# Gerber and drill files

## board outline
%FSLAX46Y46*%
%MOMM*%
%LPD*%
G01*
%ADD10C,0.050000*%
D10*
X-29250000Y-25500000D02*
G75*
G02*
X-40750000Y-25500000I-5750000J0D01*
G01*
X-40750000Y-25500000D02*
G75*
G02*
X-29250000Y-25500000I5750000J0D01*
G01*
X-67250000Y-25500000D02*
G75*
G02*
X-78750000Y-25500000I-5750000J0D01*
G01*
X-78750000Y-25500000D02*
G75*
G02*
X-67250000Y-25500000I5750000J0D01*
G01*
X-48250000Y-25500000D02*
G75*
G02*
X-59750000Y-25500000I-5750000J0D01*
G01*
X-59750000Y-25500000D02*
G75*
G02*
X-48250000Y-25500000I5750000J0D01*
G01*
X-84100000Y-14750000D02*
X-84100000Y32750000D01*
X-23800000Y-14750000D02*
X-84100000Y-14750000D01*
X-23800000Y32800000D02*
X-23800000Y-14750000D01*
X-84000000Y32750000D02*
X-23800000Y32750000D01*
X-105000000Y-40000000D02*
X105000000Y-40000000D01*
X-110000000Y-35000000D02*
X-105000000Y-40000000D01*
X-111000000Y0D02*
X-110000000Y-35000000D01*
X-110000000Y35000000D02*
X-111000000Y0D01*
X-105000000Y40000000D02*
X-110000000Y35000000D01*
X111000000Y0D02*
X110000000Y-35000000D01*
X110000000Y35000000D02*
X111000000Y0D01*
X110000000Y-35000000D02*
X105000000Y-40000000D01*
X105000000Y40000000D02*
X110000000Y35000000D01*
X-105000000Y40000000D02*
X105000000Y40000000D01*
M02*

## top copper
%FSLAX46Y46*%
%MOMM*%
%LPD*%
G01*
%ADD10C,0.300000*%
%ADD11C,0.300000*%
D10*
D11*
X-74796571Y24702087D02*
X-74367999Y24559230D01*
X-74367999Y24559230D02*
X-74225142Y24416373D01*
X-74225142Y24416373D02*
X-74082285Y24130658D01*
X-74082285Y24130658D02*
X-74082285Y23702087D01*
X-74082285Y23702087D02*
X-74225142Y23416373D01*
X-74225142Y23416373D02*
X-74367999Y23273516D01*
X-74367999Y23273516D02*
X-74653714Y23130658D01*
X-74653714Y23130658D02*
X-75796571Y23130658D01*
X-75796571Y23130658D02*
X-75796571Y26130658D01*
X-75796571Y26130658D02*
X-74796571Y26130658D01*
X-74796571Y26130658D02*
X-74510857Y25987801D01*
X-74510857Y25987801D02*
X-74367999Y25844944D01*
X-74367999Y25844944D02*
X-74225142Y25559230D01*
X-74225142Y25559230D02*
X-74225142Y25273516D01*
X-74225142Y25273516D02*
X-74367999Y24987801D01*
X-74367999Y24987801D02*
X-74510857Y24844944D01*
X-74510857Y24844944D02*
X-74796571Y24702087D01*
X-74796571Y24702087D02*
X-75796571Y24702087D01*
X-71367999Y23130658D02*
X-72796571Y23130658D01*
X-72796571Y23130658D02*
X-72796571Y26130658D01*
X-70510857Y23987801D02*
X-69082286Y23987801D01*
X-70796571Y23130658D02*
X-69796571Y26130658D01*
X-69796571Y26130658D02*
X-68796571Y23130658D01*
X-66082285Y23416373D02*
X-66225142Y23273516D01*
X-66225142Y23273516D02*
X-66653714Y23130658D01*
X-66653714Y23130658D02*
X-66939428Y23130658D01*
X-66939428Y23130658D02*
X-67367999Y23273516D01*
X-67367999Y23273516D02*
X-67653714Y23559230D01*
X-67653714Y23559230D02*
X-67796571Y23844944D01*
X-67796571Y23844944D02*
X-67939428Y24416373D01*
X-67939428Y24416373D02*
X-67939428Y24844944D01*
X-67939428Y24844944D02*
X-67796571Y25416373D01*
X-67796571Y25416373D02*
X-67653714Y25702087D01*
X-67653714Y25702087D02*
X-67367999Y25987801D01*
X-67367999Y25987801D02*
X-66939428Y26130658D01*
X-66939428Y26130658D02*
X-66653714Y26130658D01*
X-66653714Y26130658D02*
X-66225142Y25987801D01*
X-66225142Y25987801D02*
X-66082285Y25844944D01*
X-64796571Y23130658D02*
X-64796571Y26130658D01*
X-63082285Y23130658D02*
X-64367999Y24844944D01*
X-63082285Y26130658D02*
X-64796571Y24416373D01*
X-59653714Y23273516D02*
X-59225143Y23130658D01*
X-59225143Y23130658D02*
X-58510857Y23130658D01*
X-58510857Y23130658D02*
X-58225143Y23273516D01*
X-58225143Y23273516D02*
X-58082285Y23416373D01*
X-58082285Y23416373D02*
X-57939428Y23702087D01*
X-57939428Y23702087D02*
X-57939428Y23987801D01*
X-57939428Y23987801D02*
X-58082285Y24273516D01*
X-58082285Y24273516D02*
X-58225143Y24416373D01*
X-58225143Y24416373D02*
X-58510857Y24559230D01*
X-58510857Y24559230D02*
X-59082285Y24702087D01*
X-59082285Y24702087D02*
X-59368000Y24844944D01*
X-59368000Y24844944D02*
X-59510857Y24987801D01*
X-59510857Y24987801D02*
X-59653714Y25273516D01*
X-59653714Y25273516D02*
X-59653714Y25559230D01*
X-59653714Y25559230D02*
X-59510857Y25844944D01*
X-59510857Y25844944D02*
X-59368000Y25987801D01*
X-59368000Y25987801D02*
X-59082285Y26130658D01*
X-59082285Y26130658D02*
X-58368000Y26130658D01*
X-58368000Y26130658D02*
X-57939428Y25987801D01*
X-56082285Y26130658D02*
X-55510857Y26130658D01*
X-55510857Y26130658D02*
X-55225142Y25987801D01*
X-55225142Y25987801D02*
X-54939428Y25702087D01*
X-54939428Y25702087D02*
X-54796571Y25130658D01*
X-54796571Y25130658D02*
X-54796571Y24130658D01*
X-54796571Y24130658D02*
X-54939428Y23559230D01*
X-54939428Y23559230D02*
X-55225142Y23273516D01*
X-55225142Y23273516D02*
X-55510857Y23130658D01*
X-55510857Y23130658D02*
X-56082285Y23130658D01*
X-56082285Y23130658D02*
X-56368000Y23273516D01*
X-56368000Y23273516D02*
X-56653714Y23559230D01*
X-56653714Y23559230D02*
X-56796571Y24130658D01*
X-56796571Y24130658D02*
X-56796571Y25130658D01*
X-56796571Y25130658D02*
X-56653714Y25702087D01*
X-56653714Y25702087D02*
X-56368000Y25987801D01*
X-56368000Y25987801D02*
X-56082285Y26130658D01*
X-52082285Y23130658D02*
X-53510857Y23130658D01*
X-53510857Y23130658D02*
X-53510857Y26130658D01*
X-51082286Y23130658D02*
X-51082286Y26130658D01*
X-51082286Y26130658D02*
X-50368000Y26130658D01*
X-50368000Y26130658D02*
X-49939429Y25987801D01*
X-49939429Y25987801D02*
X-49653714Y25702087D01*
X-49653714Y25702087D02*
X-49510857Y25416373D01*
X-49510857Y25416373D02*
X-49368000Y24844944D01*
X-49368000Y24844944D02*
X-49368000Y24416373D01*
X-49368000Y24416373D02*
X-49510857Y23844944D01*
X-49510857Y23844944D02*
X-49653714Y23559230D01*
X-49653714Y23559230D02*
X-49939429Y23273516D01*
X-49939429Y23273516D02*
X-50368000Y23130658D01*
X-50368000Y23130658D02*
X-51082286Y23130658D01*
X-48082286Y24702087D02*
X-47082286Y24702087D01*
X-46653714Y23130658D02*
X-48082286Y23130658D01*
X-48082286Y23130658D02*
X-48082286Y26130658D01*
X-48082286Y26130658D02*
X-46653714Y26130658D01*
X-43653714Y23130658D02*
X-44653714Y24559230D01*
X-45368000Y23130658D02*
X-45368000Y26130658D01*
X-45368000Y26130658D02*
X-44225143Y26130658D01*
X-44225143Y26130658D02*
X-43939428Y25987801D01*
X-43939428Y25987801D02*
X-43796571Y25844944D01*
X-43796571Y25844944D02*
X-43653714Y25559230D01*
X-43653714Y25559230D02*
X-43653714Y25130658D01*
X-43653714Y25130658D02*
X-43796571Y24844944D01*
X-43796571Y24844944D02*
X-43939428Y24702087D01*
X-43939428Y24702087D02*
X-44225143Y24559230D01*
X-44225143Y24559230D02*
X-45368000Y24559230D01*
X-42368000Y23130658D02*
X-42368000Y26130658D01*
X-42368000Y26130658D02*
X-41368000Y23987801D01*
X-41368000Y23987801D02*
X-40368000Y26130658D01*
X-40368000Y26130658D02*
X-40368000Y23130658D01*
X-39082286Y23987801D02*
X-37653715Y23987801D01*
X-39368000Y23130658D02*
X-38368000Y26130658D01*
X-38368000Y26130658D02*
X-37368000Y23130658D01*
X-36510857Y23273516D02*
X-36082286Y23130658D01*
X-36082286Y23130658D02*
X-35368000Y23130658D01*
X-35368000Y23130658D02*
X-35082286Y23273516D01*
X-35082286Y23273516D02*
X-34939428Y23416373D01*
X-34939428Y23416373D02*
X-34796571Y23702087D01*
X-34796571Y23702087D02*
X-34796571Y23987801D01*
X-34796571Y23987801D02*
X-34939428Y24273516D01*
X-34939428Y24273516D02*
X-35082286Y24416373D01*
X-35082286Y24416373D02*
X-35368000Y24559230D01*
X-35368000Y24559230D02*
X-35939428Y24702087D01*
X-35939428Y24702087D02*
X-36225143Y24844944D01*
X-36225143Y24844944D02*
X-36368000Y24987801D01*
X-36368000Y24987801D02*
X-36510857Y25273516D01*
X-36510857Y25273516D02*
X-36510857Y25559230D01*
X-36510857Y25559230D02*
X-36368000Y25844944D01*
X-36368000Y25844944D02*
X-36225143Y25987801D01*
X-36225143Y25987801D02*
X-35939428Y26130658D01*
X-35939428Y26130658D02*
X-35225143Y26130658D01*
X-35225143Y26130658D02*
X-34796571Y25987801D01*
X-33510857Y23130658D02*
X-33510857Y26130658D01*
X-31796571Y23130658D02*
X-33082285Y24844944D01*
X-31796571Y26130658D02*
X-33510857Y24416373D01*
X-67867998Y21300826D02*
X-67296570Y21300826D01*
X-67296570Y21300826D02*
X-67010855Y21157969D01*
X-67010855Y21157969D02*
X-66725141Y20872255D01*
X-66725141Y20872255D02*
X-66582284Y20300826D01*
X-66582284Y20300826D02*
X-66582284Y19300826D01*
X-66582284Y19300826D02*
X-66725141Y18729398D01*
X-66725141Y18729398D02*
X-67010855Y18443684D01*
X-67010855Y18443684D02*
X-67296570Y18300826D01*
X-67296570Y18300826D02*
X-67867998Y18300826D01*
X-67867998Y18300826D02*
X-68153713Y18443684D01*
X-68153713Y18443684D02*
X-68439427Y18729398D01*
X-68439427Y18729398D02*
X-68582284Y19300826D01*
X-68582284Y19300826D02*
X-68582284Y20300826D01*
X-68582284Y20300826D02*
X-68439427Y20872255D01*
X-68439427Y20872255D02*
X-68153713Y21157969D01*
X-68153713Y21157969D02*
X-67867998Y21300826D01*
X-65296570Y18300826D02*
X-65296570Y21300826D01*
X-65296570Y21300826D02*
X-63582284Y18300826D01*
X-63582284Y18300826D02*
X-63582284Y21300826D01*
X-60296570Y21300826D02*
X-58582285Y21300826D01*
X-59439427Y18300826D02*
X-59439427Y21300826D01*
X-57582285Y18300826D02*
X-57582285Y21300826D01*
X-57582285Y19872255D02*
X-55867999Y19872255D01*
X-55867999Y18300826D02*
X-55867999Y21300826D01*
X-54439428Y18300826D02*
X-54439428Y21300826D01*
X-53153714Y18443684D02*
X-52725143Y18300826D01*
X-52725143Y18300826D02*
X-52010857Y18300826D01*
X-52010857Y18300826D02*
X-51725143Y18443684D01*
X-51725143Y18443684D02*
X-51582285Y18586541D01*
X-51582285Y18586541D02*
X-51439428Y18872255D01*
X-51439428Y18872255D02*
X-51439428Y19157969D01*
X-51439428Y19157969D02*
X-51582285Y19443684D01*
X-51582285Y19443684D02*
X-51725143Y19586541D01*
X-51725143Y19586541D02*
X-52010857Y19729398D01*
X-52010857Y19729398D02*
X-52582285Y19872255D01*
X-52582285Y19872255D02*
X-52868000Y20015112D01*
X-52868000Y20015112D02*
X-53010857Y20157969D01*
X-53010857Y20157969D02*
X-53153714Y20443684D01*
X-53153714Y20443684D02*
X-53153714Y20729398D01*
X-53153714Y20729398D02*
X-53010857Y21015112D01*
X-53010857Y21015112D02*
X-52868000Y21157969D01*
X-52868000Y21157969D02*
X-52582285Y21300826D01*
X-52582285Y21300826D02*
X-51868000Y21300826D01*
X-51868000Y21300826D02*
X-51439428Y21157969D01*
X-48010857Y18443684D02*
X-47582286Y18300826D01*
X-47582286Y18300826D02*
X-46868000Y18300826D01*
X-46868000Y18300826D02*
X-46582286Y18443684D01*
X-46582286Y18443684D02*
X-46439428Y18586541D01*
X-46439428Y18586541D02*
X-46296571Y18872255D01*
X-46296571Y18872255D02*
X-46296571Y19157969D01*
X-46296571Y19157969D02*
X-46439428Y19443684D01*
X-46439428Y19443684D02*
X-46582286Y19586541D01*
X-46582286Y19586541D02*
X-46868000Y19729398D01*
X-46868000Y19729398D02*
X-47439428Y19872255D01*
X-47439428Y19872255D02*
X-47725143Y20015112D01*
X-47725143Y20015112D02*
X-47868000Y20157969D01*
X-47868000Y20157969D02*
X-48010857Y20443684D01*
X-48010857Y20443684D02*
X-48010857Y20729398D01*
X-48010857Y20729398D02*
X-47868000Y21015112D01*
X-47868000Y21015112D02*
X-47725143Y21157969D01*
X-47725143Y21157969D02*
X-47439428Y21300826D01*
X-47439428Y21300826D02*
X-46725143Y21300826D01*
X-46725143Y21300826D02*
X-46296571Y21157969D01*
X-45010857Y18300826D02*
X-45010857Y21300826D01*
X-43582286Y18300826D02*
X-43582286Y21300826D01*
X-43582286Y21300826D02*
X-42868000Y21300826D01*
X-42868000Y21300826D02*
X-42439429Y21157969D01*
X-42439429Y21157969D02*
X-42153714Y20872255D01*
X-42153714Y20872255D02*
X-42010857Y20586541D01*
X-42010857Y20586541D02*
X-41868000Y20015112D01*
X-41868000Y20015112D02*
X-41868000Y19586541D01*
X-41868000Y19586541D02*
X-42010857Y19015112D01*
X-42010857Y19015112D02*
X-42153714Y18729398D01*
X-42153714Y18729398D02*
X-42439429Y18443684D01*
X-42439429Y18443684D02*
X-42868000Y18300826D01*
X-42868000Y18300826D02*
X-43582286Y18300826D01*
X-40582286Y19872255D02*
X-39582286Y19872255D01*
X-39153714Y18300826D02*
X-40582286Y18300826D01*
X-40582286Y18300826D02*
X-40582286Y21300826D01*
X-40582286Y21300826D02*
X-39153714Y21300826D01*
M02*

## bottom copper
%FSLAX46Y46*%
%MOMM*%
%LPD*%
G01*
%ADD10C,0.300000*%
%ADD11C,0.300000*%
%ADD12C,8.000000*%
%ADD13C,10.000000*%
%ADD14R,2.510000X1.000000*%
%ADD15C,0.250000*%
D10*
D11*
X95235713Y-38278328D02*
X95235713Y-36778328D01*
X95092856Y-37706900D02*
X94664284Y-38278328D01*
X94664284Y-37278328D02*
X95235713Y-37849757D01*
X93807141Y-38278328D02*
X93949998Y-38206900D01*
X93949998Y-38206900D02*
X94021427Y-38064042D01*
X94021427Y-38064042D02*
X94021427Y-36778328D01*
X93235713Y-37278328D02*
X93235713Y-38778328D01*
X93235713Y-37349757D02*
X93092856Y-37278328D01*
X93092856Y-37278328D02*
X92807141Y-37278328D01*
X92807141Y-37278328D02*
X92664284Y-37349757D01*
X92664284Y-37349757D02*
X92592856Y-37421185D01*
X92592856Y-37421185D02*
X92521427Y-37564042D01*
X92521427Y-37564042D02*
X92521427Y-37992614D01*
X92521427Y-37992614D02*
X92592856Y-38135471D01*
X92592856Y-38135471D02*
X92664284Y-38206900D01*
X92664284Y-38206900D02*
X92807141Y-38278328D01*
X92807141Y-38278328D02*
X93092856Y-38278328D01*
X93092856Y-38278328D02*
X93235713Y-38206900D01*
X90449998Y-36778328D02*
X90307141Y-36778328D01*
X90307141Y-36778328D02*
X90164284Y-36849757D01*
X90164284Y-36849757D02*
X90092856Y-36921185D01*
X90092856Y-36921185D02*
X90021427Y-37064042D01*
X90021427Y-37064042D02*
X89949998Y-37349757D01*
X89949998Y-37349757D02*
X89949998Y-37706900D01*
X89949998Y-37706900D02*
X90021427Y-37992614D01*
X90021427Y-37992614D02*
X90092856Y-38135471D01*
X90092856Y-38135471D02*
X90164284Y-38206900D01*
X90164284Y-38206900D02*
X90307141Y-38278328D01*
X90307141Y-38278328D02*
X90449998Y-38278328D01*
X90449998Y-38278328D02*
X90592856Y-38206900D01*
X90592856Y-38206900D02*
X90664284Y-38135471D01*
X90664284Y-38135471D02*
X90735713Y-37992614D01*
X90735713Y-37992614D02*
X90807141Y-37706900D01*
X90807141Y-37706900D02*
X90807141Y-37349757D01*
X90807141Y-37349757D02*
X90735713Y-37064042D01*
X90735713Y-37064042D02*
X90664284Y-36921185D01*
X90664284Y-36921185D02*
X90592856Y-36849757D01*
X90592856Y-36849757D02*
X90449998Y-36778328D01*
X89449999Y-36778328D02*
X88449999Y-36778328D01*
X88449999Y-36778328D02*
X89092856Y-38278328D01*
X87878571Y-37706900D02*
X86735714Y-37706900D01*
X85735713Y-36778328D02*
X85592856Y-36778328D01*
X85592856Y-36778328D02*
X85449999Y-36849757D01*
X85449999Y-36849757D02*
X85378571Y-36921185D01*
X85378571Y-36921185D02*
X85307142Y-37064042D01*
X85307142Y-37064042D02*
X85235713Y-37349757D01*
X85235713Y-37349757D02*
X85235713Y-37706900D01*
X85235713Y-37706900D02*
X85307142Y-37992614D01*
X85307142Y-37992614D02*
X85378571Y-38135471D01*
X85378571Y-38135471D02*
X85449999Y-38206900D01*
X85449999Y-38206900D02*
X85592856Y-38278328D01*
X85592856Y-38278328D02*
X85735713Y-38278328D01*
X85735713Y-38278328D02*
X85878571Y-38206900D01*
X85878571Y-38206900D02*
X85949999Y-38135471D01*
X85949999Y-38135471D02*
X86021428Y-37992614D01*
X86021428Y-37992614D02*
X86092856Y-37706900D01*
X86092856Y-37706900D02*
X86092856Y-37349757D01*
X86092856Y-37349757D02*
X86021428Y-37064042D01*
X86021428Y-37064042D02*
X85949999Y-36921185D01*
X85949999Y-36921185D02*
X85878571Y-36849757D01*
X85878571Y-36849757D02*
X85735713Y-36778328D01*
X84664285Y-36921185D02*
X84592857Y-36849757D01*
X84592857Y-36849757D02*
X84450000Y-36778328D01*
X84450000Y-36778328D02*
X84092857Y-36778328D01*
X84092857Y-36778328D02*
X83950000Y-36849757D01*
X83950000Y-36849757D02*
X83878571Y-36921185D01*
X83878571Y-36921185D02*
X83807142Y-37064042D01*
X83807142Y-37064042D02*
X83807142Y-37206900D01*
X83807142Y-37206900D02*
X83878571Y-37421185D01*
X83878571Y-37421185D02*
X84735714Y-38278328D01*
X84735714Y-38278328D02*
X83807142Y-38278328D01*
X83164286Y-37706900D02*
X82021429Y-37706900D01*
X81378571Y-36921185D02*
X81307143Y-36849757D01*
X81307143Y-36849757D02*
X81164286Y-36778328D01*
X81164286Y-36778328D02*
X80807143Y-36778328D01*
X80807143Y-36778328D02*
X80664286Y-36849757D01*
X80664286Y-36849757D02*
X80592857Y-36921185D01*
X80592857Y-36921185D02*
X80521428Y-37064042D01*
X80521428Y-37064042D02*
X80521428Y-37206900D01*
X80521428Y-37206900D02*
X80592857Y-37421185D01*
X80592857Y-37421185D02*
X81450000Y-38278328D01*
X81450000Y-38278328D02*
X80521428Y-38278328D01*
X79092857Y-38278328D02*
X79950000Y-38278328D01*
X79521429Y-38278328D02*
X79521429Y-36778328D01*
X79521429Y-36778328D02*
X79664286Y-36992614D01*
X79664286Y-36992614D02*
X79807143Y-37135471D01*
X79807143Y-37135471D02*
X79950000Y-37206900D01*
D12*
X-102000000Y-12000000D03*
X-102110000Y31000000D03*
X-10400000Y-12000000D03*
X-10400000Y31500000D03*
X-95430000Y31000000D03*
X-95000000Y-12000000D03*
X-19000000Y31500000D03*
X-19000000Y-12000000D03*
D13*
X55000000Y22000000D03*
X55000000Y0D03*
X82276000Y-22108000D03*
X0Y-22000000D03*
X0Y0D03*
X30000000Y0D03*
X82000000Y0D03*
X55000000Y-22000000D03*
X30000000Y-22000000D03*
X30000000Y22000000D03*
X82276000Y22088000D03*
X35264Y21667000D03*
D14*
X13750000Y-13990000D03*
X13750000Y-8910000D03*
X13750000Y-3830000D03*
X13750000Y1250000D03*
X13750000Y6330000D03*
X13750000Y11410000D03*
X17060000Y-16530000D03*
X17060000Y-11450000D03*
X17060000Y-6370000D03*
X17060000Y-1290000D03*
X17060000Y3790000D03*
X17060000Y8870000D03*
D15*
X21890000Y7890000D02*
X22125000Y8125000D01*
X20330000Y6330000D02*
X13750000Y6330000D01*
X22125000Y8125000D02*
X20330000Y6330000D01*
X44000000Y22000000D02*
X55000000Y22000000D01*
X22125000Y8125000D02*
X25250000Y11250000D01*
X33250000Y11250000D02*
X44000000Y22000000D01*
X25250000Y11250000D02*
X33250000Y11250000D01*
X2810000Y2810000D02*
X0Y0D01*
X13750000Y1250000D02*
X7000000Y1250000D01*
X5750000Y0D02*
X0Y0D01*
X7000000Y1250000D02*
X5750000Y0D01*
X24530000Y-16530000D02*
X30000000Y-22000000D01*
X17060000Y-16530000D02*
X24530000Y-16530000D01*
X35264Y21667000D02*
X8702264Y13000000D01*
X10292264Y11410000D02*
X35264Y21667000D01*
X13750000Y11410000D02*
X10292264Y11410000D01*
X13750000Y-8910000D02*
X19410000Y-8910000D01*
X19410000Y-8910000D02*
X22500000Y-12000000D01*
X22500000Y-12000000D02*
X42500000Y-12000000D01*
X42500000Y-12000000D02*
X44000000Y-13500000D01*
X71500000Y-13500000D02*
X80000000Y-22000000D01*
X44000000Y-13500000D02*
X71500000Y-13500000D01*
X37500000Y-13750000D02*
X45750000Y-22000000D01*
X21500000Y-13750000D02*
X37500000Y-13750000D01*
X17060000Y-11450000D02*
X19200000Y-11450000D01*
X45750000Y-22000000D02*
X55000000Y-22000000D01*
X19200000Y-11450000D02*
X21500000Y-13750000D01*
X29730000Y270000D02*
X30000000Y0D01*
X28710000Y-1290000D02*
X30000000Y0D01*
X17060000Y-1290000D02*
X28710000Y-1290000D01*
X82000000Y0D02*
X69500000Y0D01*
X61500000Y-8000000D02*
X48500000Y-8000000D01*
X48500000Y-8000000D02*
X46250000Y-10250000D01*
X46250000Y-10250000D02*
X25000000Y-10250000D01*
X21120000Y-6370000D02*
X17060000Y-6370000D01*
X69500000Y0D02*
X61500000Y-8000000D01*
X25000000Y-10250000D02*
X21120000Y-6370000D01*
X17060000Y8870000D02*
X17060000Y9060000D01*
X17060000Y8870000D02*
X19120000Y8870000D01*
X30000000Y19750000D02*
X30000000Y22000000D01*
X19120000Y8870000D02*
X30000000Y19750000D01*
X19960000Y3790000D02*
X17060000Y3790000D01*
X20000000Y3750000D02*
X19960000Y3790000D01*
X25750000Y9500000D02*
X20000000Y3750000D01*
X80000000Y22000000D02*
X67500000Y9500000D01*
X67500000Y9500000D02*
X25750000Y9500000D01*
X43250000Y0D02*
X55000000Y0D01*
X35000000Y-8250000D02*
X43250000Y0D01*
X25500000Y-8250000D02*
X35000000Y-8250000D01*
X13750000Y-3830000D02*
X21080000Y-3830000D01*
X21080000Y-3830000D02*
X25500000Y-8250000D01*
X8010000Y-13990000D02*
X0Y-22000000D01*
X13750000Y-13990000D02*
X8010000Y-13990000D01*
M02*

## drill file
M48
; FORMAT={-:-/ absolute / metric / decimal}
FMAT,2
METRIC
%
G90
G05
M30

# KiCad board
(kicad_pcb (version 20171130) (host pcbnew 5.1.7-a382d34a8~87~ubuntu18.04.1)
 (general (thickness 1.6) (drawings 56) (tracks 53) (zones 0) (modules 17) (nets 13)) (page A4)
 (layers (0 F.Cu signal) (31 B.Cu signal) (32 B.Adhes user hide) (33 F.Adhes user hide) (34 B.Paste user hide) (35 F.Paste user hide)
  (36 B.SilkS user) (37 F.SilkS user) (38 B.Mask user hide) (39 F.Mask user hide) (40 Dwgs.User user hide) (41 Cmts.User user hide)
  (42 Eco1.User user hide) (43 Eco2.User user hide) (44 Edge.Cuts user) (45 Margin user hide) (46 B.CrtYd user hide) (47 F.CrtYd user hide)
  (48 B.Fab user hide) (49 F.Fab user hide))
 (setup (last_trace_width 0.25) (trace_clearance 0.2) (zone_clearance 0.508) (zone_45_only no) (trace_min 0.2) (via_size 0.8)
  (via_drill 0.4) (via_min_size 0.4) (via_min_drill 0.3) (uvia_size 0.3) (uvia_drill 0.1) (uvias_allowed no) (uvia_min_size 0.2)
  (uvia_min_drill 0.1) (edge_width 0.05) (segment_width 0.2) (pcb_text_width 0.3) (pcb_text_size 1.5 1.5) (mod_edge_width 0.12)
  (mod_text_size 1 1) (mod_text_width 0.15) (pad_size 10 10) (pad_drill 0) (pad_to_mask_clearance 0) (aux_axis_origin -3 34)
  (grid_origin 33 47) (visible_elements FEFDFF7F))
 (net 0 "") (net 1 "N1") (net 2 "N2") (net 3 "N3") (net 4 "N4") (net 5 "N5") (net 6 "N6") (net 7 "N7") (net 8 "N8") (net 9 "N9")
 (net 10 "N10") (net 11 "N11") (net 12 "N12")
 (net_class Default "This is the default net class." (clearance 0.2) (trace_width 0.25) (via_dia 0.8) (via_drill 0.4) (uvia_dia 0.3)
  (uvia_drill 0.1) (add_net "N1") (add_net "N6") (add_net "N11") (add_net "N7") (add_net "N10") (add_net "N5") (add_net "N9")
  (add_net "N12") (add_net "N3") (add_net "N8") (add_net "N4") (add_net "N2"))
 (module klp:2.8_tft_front (layer F.Cu) (at -54 -9 270)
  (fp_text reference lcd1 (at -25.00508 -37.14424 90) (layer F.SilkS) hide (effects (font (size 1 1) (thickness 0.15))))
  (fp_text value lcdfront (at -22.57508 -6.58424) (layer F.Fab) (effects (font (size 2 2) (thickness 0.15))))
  (pad "" smd circle (at 21 48 270) (size 8 8) (layers B.Cu F.Paste F.Mask))
  (pad "" smd circle (at -22 48.11 270) (size 8 8) (layers B.Cu F.Paste F.Mask))
  (pad "" smd circle (at 21 -43.6 270) (size 8 8) (layers B.Cu F.Paste F.Mask))
  (pad "" smd circle (at -22.5 -43.6 270) (size 8 8) (layers B.Cu F.Paste F.Mask))
  (pad "" smd circle (at -22 41.43 270) (size 8 8) (layers B.Cu F.Paste F.Mask))
  (pad "" smd circle (at 21 41 270) (size 8 8) (layers B.Cu F.Paste F.Mask))
  (pad "" smd circle (at -22.5 -35 270) (size 8 8) (layers B.Cu F.Paste F.Mask))
  (pad "" smd circle (at 21 -35 270) (size 8 8) (layers B.Cu F.Paste F.Mask)))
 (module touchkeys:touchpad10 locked (layer B.Cu) (at 55 -22)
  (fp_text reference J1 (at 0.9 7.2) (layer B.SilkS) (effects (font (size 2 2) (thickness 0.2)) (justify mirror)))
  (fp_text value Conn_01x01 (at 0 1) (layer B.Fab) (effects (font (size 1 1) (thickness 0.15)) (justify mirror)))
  (pad 1 smd circle (at 0 0) (size 10 10) (layers B.Cu B.Paste B.Mask) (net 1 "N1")))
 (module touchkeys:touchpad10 (layer B.Cu) (at 55 0)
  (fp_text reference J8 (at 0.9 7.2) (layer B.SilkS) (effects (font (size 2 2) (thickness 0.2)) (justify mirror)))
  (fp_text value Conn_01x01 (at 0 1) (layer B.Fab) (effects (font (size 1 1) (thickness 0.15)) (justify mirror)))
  (pad 1 smd circle (at 0 0) (size 10 10) (layers B.Cu B.Paste B.Mask) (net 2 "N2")))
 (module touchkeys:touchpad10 (layer B.Cu) (at 82.276 22.108)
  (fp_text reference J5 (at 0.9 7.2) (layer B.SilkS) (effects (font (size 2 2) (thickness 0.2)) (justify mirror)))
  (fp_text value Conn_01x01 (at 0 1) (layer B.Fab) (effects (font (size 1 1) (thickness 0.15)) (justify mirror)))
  (pad 1 smd circle (at 0 0) (size 10 10) (layers B.Cu B.Paste B.Mask) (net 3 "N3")))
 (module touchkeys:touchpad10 (layer B.Cu) (at 0 22)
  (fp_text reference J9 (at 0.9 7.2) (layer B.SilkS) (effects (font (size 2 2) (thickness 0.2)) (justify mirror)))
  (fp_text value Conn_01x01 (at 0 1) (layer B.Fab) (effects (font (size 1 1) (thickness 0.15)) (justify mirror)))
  (pad 1 smd circle (at 0 0) (size 10 10) (layers B.Cu B.Paste B.Mask) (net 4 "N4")))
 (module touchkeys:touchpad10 (layer B.Cu) (at 0 0)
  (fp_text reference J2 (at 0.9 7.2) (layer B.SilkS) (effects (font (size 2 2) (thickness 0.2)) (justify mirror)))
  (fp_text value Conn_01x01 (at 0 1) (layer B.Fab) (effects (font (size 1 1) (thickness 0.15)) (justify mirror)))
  (pad 1 smd circle (at 0 0) (size 10 10) (layers B.Cu B.Paste B.Mask) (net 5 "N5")))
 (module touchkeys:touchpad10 (layer B.Cu) (at 30 0)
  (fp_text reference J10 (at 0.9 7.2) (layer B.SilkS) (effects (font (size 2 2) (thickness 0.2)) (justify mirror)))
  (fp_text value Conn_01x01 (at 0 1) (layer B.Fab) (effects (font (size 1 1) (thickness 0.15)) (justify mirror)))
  (pad 1 smd circle (at 0 0) (size 10 10) (layers B.Cu B.Paste B.Mask) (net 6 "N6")))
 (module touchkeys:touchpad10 (layer B.Cu) (at 82 0)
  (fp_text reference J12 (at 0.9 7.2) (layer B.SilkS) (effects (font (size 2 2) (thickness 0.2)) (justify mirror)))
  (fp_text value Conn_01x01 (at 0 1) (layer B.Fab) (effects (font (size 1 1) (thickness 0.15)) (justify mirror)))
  (pad 1 smd circle (at 0 0) (size 10 10) (layers B.Cu B.Paste B.Mask) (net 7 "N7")))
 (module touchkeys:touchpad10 (layer B.Cu) (at 55 22)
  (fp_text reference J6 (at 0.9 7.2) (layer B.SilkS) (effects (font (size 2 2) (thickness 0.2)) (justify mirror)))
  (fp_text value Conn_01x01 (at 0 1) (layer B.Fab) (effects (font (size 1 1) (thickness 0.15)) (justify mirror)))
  (pad 1 smd circle (at 0 0) (size 10 10) (layers B.Cu B.Paste B.Mask) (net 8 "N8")))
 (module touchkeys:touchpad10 (layer B.Cu) (at 30 22)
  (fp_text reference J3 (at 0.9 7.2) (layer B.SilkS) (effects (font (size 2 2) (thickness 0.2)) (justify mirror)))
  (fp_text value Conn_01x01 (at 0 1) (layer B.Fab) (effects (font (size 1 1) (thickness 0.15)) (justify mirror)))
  (pad 1 smd circle (at 0 0) (size 10 10) (layers B.Cu B.Paste B.Mask) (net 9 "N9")))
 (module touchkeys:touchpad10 (layer B.Cu) (at 30 -22)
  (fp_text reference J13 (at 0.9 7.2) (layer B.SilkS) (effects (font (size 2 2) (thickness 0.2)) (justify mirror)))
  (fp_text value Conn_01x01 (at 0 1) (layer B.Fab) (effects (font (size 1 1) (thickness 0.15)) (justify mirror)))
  (pad 1 smd circle (at 0 0) (size 10 10) (layers B.Cu B.Paste B.Mask) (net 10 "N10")))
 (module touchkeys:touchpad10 (layer B.Cu) (at 82.276 -22.088)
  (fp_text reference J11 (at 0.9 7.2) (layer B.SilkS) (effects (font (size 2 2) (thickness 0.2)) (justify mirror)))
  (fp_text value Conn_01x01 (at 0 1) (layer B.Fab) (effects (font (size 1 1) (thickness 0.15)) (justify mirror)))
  (pad 1 smd circle (at 0 0) (size 10 10) (layers B.Cu B.Paste B.Mask) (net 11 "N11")))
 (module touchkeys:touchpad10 (layer B.Cu) (at 0.035264 -21.667)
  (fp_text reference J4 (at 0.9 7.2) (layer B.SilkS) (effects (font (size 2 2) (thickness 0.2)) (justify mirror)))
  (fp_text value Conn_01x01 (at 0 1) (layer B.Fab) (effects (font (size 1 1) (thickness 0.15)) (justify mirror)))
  (pad 1 smd circle (at 0 0) (size 10 10) (layers B.Cu B.Paste B.Mask) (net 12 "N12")))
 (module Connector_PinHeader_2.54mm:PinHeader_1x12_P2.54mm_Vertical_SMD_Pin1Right (layer B.Cu) (at 15.405 2.56 180)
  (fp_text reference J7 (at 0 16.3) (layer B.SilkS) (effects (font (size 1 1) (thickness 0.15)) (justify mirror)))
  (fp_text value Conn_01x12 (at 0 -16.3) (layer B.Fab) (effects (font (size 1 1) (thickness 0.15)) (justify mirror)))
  (pad 11 smd rect (at 1.655 -11.43 180) (size 2.51 1) (layers B.Cu B.Paste B.Mask) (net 4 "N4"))
  (pad 9 smd rect (at 1.655 -6.35 180) (size 2.51 1) (layers B.Cu B.Paste B.Mask) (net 3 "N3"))
  (pad 7 smd rect (at 1.655 -1.27 180) (size 2.51 1) (layers B.Cu B.Paste B.Mask) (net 2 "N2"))
  (pad 5 smd rect (at 1.655 3.81 180) (size 2.51 1) (layers B.Cu B.Paste B.Mask) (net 5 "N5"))
  (pad 3 smd rect (at 1.655 8.89 180) (size 2.51 1) (layers B.Cu B.Paste B.Mask) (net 1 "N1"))
  (pad 1 smd rect (at 1.655 13.97 180) (size 2.51 1) (layers B.Cu B.Paste B.Mask) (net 12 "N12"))
  (pad 12 smd rect (at -1.655 -13.97 180) (size 2.51 1) (layers B.Cu B.Paste B.Mask) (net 9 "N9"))
  (pad 10 smd rect (at -1.655 -8.89 180) (size 2.51 1) (layers B.Cu B.Paste B.Mask) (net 8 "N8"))
  (pad 8 smd rect (at -1.655 -3.81 180) (size 2.51 1) (layers B.Cu B.Paste B.Mask) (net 7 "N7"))
  (pad 6 smd rect (at -1.655 1.27 180) (size 2.51 1) (layers B.Cu B.Paste B.Mask) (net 6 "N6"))
  (pad 4 smd rect (at -1.655 6.35 180) (size 2.51 1) (layers B.Cu B.Paste B.Mask) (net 11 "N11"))
  (pad 2 smd rect (at -1.655 11.43 180) (size 2.51 1) (layers B.Cu B.Paste B.Mask) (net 10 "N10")))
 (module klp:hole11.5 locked (layer F.Cu) (at -35 25.5)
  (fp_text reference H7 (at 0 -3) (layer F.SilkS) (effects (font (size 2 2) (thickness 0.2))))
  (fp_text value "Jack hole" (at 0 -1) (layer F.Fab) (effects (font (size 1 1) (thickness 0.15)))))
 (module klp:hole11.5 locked (layer F.Cu) (at -54 25.5)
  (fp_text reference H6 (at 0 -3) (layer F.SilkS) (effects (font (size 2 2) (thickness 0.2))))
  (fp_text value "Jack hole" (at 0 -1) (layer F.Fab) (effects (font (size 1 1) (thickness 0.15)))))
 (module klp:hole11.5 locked (layer F.Cu) (at -73 25.5)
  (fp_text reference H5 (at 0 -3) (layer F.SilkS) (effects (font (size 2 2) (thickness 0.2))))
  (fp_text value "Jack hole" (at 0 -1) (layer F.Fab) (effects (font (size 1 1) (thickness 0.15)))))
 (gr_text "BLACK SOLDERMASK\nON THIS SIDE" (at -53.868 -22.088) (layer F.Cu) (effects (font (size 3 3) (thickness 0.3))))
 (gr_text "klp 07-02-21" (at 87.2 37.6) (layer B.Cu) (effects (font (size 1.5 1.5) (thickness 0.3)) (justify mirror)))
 (gr_circle (center -35 25.5) (end -29.25 25.5) (layer Edge.Cuts) (width 0.05))
 (gr_circle (center -73 25.5) (end -67.25 25.5) (layer Edge.Cuts) (width 0.05))
 (gr_circle (center -54 25.5) (end -48.25 25.5) (layer Edge.Cuts) (width 0.05))
 (gr_line (start -84.1 14.75) (end -84.1 -32.75) (layer Edge.Cuts) (width 0.05))
 (gr_line (start -23.8 14.75) (end -84.1 14.75) (layer Edge.Cuts) (width 0.05))
 (gr_line (start -23.8 -32.8) (end -23.8 14.75) (layer Edge.Cuts) (width 0.05))
 (gr_line (start -84 -32.75) (end -23.8 -32.75) (layer Edge.Cuts) (width 0.05))
 (gr_line (start -105 40) (end 105 40) (layer Edge.Cuts) (width 0.05))
 (gr_line (start -110 35) (end -105 40) (layer Edge.Cuts) (width 0.05))
 (gr_line (start -111 0) (end -110 35) (layer Edge.Cuts) (width 0.05))
 (gr_line (start -110 -35) (end -111 0) (layer Edge.Cuts) (width 0.05))
 (gr_line (start -105 -40) (end -110 -35) (layer Edge.Cuts) (width 0.05))
 (gr_line (start 111 0) (end 110 35) (layer Edge.Cuts) (width 0.05))
 (gr_line (start 110 -35) (end 111 0) (layer Edge.Cuts) (width 0.05))
 (gr_line (start 110 35) (end 105 40) (layer Edge.Cuts) (width 0.05))
 (gr_line (start 105 -40) (end 110 -35) (layer Edge.Cuts) (width 0.05))
 (gr_line (start -105 -40) (end 105 -40) (layer Edge.Cuts) (width 0.05))
 (segment (start 21.89 -7.89) (end 22.125 -8.125) (width 0.25) (layer B.Cu) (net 1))
 (segment (start 20.33 -6.33) (end 13.75 -6.33) (width 0.25) (layer B.Cu) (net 1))
 (segment (start 22.125 -8.125) (end 20.33 -6.33) (width 0.25) (layer B.Cu) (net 1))
 (segment (start 44 -22) (end 55 -22) (width 0.25) (layer B.Cu) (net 1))
 (segment (start 22.125 -8.125) (end 25.25 -11.25) (width 0.25) (layer B.Cu) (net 1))
 (segment (start 33.25 -11.25) (end 44 -22) (width 0.25) (layer B.Cu) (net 1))
 (segment (start 25.25 -11.25) (end 33.25 -11.25) (width 0.25) (layer B.Cu) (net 1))
 (segment (start 2.81 -2.81) (end 0 0) (width 0.25) (layer B.Cu) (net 5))
 (segment (start 13.75 -1.25) (end 7 -1.25) (width 0.25) (layer B.Cu) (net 5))
 (segment (start 5.75 0) (end 0 0) (width 0.25) (layer B.Cu) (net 5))
 (segment (start 7 -1.25) (end 5.75 0) (width 0.25) (layer B.Cu) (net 5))
 (segment (start 24.53 16.53) (end 30 22) (width 0.25) (layer B.Cu) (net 9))
 (segment (start 17.06 16.53) (end 24.53 16.53) (width 0.25) (layer B.Cu) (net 9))
 (segment (start 0.035264 -21.667) (end 8.702264 -13) (width 0.25) (layer B.Cu) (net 12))
 (segment (start 10.292264 -11.41) (end 0.035264 -21.667) (width 0.25) (layer B.Cu) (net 12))
 (segment (start 13.75 -11.41) (end 10.292264 -11.41) (width 0.25) (layer B.Cu) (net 12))
 (segment (start 13.75 8.91) (end 19.41 8.91) (width 0.25) (layer B.Cu) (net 3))
 (segment (start 19.41 8.91) (end 22.5 12) (width 0.25) (layer B.Cu) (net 3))
 (segment (start 22.5 12) (end 42.5 12) (width 0.25) (layer B.Cu) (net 3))
 (segment (start 42.5 12) (end 44 13.5) (width 0.25) (layer B.Cu) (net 3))
 (segment (start 71.5 13.5) (end 80 22) (width 0.25) (layer B.Cu) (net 3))
 (segment (start 44 13.5) (end 71.5 13.5) (width 0.25) (layer B.Cu) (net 3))
 (segment (start 37.5 13.75) (end 45.75 22) (width 0.25) (layer B.Cu) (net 8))
 (segment (start 21.5 13.75) (end 37.5 13.75) (width 0.25) (layer B.Cu) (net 8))
 (segment (start 17.06 11.45) (end 19.2 11.45) (width 0.25) (layer B.Cu) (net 8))
 (segment (start 45.75 22) (end 55 22) (width 0.25) (layer B.Cu) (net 8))
 (segment (start 19.2 11.45) (end 21.5 13.75) (width 0.25) (layer B.Cu) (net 8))
 (segment (start 29.73 -0.27) (end 30 0) (width 0.25) (layer B.Cu) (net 6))
 (segment (start 28.71 1.29) (end 30 0) (width 0.25) (layer B.Cu) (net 6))
 (segment (start 17.06 1.29) (end 28.71 1.29) (width 0.25) (layer B.Cu) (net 6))
 (segment (start 82 0) (end 69.5 0) (width 0.25) (layer B.Cu) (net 7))
 (segment (start 61.5 8) (end 48.5 8) (width 0.25) (layer B.Cu) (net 7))
 (segment (start 48.5 8) (end 46.25 10.25) (width 0.25) (layer B.Cu) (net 7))
 (segment (start 46.25 10.25) (end 25 10.25) (width 0.25) (layer B.Cu) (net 7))
 (segment (start 21.12 6.37) (end 17.06 6.37) (width 0.25) (layer B.Cu) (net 7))
 (segment (start 69.5 0) (end 61.5 8) (width 0.25) (layer B.Cu) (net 7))
 (segment (start 25 10.25) (end 21.12 6.37) (width 0.25) (layer B.Cu) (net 7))
 (segment (start 17.06 -8.87) (end 17.06 -9.06) (width 0.25) (layer B.Cu) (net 10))
 (segment (start 17.06 -8.87) (end 19.12 -8.87) (width 0.25) (layer B.Cu) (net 10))
 (segment (start 30 -19.75) (end 30 -22) (width 0.25) (layer B.Cu) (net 10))
 (segment (start 19.12 -8.87) (end 30 -19.75) (width 0.25) (layer B.Cu) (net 10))
 (segment (start 19.96 -3.79) (end 17.06 -3.79) (width 0.25) (layer B.Cu) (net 11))
 (segment (start 20 -3.75) (end 19.96 -3.79) (width 0.25) (layer B.Cu) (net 11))
 (segment (start 25.75 -9.5) (end 20 -3.75) (width 0.25) (layer B.Cu) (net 11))
 (segment (start 80 -22) (end 67.5 -9.5) (width 0.25) (layer B.Cu) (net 11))
 (segment (start 67.5 -9.5) (end 25.75 -9.5) (width 0.25) (layer B.Cu) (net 11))
 (segment (start 43.25 0) (end 55 0) (width 0.25) (layer B.Cu) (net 2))
 (segment (start 35 8.25) (end 43.25 0) (width 0.25) (layer B.Cu) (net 2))
 (segment (start 25.5 8.25) (end 35 8.25) (width 0.25) (layer B.Cu) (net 2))
 (segment (start 13.75 3.83) (end 21.08 3.83) (width 0.25) (layer B.Cu) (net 2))
 (segment (start 21.08 3.83) (end 25.5 8.25) (width 0.25) (layer B.Cu) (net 2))
 (segment (start 8.01 13.99) (end 0 22) (width 0.25) (layer B.Cu) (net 4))
 (segment (start 13.75 13.99) (end 8.01 13.99) (width 0.25) (layer B.Cu) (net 4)))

